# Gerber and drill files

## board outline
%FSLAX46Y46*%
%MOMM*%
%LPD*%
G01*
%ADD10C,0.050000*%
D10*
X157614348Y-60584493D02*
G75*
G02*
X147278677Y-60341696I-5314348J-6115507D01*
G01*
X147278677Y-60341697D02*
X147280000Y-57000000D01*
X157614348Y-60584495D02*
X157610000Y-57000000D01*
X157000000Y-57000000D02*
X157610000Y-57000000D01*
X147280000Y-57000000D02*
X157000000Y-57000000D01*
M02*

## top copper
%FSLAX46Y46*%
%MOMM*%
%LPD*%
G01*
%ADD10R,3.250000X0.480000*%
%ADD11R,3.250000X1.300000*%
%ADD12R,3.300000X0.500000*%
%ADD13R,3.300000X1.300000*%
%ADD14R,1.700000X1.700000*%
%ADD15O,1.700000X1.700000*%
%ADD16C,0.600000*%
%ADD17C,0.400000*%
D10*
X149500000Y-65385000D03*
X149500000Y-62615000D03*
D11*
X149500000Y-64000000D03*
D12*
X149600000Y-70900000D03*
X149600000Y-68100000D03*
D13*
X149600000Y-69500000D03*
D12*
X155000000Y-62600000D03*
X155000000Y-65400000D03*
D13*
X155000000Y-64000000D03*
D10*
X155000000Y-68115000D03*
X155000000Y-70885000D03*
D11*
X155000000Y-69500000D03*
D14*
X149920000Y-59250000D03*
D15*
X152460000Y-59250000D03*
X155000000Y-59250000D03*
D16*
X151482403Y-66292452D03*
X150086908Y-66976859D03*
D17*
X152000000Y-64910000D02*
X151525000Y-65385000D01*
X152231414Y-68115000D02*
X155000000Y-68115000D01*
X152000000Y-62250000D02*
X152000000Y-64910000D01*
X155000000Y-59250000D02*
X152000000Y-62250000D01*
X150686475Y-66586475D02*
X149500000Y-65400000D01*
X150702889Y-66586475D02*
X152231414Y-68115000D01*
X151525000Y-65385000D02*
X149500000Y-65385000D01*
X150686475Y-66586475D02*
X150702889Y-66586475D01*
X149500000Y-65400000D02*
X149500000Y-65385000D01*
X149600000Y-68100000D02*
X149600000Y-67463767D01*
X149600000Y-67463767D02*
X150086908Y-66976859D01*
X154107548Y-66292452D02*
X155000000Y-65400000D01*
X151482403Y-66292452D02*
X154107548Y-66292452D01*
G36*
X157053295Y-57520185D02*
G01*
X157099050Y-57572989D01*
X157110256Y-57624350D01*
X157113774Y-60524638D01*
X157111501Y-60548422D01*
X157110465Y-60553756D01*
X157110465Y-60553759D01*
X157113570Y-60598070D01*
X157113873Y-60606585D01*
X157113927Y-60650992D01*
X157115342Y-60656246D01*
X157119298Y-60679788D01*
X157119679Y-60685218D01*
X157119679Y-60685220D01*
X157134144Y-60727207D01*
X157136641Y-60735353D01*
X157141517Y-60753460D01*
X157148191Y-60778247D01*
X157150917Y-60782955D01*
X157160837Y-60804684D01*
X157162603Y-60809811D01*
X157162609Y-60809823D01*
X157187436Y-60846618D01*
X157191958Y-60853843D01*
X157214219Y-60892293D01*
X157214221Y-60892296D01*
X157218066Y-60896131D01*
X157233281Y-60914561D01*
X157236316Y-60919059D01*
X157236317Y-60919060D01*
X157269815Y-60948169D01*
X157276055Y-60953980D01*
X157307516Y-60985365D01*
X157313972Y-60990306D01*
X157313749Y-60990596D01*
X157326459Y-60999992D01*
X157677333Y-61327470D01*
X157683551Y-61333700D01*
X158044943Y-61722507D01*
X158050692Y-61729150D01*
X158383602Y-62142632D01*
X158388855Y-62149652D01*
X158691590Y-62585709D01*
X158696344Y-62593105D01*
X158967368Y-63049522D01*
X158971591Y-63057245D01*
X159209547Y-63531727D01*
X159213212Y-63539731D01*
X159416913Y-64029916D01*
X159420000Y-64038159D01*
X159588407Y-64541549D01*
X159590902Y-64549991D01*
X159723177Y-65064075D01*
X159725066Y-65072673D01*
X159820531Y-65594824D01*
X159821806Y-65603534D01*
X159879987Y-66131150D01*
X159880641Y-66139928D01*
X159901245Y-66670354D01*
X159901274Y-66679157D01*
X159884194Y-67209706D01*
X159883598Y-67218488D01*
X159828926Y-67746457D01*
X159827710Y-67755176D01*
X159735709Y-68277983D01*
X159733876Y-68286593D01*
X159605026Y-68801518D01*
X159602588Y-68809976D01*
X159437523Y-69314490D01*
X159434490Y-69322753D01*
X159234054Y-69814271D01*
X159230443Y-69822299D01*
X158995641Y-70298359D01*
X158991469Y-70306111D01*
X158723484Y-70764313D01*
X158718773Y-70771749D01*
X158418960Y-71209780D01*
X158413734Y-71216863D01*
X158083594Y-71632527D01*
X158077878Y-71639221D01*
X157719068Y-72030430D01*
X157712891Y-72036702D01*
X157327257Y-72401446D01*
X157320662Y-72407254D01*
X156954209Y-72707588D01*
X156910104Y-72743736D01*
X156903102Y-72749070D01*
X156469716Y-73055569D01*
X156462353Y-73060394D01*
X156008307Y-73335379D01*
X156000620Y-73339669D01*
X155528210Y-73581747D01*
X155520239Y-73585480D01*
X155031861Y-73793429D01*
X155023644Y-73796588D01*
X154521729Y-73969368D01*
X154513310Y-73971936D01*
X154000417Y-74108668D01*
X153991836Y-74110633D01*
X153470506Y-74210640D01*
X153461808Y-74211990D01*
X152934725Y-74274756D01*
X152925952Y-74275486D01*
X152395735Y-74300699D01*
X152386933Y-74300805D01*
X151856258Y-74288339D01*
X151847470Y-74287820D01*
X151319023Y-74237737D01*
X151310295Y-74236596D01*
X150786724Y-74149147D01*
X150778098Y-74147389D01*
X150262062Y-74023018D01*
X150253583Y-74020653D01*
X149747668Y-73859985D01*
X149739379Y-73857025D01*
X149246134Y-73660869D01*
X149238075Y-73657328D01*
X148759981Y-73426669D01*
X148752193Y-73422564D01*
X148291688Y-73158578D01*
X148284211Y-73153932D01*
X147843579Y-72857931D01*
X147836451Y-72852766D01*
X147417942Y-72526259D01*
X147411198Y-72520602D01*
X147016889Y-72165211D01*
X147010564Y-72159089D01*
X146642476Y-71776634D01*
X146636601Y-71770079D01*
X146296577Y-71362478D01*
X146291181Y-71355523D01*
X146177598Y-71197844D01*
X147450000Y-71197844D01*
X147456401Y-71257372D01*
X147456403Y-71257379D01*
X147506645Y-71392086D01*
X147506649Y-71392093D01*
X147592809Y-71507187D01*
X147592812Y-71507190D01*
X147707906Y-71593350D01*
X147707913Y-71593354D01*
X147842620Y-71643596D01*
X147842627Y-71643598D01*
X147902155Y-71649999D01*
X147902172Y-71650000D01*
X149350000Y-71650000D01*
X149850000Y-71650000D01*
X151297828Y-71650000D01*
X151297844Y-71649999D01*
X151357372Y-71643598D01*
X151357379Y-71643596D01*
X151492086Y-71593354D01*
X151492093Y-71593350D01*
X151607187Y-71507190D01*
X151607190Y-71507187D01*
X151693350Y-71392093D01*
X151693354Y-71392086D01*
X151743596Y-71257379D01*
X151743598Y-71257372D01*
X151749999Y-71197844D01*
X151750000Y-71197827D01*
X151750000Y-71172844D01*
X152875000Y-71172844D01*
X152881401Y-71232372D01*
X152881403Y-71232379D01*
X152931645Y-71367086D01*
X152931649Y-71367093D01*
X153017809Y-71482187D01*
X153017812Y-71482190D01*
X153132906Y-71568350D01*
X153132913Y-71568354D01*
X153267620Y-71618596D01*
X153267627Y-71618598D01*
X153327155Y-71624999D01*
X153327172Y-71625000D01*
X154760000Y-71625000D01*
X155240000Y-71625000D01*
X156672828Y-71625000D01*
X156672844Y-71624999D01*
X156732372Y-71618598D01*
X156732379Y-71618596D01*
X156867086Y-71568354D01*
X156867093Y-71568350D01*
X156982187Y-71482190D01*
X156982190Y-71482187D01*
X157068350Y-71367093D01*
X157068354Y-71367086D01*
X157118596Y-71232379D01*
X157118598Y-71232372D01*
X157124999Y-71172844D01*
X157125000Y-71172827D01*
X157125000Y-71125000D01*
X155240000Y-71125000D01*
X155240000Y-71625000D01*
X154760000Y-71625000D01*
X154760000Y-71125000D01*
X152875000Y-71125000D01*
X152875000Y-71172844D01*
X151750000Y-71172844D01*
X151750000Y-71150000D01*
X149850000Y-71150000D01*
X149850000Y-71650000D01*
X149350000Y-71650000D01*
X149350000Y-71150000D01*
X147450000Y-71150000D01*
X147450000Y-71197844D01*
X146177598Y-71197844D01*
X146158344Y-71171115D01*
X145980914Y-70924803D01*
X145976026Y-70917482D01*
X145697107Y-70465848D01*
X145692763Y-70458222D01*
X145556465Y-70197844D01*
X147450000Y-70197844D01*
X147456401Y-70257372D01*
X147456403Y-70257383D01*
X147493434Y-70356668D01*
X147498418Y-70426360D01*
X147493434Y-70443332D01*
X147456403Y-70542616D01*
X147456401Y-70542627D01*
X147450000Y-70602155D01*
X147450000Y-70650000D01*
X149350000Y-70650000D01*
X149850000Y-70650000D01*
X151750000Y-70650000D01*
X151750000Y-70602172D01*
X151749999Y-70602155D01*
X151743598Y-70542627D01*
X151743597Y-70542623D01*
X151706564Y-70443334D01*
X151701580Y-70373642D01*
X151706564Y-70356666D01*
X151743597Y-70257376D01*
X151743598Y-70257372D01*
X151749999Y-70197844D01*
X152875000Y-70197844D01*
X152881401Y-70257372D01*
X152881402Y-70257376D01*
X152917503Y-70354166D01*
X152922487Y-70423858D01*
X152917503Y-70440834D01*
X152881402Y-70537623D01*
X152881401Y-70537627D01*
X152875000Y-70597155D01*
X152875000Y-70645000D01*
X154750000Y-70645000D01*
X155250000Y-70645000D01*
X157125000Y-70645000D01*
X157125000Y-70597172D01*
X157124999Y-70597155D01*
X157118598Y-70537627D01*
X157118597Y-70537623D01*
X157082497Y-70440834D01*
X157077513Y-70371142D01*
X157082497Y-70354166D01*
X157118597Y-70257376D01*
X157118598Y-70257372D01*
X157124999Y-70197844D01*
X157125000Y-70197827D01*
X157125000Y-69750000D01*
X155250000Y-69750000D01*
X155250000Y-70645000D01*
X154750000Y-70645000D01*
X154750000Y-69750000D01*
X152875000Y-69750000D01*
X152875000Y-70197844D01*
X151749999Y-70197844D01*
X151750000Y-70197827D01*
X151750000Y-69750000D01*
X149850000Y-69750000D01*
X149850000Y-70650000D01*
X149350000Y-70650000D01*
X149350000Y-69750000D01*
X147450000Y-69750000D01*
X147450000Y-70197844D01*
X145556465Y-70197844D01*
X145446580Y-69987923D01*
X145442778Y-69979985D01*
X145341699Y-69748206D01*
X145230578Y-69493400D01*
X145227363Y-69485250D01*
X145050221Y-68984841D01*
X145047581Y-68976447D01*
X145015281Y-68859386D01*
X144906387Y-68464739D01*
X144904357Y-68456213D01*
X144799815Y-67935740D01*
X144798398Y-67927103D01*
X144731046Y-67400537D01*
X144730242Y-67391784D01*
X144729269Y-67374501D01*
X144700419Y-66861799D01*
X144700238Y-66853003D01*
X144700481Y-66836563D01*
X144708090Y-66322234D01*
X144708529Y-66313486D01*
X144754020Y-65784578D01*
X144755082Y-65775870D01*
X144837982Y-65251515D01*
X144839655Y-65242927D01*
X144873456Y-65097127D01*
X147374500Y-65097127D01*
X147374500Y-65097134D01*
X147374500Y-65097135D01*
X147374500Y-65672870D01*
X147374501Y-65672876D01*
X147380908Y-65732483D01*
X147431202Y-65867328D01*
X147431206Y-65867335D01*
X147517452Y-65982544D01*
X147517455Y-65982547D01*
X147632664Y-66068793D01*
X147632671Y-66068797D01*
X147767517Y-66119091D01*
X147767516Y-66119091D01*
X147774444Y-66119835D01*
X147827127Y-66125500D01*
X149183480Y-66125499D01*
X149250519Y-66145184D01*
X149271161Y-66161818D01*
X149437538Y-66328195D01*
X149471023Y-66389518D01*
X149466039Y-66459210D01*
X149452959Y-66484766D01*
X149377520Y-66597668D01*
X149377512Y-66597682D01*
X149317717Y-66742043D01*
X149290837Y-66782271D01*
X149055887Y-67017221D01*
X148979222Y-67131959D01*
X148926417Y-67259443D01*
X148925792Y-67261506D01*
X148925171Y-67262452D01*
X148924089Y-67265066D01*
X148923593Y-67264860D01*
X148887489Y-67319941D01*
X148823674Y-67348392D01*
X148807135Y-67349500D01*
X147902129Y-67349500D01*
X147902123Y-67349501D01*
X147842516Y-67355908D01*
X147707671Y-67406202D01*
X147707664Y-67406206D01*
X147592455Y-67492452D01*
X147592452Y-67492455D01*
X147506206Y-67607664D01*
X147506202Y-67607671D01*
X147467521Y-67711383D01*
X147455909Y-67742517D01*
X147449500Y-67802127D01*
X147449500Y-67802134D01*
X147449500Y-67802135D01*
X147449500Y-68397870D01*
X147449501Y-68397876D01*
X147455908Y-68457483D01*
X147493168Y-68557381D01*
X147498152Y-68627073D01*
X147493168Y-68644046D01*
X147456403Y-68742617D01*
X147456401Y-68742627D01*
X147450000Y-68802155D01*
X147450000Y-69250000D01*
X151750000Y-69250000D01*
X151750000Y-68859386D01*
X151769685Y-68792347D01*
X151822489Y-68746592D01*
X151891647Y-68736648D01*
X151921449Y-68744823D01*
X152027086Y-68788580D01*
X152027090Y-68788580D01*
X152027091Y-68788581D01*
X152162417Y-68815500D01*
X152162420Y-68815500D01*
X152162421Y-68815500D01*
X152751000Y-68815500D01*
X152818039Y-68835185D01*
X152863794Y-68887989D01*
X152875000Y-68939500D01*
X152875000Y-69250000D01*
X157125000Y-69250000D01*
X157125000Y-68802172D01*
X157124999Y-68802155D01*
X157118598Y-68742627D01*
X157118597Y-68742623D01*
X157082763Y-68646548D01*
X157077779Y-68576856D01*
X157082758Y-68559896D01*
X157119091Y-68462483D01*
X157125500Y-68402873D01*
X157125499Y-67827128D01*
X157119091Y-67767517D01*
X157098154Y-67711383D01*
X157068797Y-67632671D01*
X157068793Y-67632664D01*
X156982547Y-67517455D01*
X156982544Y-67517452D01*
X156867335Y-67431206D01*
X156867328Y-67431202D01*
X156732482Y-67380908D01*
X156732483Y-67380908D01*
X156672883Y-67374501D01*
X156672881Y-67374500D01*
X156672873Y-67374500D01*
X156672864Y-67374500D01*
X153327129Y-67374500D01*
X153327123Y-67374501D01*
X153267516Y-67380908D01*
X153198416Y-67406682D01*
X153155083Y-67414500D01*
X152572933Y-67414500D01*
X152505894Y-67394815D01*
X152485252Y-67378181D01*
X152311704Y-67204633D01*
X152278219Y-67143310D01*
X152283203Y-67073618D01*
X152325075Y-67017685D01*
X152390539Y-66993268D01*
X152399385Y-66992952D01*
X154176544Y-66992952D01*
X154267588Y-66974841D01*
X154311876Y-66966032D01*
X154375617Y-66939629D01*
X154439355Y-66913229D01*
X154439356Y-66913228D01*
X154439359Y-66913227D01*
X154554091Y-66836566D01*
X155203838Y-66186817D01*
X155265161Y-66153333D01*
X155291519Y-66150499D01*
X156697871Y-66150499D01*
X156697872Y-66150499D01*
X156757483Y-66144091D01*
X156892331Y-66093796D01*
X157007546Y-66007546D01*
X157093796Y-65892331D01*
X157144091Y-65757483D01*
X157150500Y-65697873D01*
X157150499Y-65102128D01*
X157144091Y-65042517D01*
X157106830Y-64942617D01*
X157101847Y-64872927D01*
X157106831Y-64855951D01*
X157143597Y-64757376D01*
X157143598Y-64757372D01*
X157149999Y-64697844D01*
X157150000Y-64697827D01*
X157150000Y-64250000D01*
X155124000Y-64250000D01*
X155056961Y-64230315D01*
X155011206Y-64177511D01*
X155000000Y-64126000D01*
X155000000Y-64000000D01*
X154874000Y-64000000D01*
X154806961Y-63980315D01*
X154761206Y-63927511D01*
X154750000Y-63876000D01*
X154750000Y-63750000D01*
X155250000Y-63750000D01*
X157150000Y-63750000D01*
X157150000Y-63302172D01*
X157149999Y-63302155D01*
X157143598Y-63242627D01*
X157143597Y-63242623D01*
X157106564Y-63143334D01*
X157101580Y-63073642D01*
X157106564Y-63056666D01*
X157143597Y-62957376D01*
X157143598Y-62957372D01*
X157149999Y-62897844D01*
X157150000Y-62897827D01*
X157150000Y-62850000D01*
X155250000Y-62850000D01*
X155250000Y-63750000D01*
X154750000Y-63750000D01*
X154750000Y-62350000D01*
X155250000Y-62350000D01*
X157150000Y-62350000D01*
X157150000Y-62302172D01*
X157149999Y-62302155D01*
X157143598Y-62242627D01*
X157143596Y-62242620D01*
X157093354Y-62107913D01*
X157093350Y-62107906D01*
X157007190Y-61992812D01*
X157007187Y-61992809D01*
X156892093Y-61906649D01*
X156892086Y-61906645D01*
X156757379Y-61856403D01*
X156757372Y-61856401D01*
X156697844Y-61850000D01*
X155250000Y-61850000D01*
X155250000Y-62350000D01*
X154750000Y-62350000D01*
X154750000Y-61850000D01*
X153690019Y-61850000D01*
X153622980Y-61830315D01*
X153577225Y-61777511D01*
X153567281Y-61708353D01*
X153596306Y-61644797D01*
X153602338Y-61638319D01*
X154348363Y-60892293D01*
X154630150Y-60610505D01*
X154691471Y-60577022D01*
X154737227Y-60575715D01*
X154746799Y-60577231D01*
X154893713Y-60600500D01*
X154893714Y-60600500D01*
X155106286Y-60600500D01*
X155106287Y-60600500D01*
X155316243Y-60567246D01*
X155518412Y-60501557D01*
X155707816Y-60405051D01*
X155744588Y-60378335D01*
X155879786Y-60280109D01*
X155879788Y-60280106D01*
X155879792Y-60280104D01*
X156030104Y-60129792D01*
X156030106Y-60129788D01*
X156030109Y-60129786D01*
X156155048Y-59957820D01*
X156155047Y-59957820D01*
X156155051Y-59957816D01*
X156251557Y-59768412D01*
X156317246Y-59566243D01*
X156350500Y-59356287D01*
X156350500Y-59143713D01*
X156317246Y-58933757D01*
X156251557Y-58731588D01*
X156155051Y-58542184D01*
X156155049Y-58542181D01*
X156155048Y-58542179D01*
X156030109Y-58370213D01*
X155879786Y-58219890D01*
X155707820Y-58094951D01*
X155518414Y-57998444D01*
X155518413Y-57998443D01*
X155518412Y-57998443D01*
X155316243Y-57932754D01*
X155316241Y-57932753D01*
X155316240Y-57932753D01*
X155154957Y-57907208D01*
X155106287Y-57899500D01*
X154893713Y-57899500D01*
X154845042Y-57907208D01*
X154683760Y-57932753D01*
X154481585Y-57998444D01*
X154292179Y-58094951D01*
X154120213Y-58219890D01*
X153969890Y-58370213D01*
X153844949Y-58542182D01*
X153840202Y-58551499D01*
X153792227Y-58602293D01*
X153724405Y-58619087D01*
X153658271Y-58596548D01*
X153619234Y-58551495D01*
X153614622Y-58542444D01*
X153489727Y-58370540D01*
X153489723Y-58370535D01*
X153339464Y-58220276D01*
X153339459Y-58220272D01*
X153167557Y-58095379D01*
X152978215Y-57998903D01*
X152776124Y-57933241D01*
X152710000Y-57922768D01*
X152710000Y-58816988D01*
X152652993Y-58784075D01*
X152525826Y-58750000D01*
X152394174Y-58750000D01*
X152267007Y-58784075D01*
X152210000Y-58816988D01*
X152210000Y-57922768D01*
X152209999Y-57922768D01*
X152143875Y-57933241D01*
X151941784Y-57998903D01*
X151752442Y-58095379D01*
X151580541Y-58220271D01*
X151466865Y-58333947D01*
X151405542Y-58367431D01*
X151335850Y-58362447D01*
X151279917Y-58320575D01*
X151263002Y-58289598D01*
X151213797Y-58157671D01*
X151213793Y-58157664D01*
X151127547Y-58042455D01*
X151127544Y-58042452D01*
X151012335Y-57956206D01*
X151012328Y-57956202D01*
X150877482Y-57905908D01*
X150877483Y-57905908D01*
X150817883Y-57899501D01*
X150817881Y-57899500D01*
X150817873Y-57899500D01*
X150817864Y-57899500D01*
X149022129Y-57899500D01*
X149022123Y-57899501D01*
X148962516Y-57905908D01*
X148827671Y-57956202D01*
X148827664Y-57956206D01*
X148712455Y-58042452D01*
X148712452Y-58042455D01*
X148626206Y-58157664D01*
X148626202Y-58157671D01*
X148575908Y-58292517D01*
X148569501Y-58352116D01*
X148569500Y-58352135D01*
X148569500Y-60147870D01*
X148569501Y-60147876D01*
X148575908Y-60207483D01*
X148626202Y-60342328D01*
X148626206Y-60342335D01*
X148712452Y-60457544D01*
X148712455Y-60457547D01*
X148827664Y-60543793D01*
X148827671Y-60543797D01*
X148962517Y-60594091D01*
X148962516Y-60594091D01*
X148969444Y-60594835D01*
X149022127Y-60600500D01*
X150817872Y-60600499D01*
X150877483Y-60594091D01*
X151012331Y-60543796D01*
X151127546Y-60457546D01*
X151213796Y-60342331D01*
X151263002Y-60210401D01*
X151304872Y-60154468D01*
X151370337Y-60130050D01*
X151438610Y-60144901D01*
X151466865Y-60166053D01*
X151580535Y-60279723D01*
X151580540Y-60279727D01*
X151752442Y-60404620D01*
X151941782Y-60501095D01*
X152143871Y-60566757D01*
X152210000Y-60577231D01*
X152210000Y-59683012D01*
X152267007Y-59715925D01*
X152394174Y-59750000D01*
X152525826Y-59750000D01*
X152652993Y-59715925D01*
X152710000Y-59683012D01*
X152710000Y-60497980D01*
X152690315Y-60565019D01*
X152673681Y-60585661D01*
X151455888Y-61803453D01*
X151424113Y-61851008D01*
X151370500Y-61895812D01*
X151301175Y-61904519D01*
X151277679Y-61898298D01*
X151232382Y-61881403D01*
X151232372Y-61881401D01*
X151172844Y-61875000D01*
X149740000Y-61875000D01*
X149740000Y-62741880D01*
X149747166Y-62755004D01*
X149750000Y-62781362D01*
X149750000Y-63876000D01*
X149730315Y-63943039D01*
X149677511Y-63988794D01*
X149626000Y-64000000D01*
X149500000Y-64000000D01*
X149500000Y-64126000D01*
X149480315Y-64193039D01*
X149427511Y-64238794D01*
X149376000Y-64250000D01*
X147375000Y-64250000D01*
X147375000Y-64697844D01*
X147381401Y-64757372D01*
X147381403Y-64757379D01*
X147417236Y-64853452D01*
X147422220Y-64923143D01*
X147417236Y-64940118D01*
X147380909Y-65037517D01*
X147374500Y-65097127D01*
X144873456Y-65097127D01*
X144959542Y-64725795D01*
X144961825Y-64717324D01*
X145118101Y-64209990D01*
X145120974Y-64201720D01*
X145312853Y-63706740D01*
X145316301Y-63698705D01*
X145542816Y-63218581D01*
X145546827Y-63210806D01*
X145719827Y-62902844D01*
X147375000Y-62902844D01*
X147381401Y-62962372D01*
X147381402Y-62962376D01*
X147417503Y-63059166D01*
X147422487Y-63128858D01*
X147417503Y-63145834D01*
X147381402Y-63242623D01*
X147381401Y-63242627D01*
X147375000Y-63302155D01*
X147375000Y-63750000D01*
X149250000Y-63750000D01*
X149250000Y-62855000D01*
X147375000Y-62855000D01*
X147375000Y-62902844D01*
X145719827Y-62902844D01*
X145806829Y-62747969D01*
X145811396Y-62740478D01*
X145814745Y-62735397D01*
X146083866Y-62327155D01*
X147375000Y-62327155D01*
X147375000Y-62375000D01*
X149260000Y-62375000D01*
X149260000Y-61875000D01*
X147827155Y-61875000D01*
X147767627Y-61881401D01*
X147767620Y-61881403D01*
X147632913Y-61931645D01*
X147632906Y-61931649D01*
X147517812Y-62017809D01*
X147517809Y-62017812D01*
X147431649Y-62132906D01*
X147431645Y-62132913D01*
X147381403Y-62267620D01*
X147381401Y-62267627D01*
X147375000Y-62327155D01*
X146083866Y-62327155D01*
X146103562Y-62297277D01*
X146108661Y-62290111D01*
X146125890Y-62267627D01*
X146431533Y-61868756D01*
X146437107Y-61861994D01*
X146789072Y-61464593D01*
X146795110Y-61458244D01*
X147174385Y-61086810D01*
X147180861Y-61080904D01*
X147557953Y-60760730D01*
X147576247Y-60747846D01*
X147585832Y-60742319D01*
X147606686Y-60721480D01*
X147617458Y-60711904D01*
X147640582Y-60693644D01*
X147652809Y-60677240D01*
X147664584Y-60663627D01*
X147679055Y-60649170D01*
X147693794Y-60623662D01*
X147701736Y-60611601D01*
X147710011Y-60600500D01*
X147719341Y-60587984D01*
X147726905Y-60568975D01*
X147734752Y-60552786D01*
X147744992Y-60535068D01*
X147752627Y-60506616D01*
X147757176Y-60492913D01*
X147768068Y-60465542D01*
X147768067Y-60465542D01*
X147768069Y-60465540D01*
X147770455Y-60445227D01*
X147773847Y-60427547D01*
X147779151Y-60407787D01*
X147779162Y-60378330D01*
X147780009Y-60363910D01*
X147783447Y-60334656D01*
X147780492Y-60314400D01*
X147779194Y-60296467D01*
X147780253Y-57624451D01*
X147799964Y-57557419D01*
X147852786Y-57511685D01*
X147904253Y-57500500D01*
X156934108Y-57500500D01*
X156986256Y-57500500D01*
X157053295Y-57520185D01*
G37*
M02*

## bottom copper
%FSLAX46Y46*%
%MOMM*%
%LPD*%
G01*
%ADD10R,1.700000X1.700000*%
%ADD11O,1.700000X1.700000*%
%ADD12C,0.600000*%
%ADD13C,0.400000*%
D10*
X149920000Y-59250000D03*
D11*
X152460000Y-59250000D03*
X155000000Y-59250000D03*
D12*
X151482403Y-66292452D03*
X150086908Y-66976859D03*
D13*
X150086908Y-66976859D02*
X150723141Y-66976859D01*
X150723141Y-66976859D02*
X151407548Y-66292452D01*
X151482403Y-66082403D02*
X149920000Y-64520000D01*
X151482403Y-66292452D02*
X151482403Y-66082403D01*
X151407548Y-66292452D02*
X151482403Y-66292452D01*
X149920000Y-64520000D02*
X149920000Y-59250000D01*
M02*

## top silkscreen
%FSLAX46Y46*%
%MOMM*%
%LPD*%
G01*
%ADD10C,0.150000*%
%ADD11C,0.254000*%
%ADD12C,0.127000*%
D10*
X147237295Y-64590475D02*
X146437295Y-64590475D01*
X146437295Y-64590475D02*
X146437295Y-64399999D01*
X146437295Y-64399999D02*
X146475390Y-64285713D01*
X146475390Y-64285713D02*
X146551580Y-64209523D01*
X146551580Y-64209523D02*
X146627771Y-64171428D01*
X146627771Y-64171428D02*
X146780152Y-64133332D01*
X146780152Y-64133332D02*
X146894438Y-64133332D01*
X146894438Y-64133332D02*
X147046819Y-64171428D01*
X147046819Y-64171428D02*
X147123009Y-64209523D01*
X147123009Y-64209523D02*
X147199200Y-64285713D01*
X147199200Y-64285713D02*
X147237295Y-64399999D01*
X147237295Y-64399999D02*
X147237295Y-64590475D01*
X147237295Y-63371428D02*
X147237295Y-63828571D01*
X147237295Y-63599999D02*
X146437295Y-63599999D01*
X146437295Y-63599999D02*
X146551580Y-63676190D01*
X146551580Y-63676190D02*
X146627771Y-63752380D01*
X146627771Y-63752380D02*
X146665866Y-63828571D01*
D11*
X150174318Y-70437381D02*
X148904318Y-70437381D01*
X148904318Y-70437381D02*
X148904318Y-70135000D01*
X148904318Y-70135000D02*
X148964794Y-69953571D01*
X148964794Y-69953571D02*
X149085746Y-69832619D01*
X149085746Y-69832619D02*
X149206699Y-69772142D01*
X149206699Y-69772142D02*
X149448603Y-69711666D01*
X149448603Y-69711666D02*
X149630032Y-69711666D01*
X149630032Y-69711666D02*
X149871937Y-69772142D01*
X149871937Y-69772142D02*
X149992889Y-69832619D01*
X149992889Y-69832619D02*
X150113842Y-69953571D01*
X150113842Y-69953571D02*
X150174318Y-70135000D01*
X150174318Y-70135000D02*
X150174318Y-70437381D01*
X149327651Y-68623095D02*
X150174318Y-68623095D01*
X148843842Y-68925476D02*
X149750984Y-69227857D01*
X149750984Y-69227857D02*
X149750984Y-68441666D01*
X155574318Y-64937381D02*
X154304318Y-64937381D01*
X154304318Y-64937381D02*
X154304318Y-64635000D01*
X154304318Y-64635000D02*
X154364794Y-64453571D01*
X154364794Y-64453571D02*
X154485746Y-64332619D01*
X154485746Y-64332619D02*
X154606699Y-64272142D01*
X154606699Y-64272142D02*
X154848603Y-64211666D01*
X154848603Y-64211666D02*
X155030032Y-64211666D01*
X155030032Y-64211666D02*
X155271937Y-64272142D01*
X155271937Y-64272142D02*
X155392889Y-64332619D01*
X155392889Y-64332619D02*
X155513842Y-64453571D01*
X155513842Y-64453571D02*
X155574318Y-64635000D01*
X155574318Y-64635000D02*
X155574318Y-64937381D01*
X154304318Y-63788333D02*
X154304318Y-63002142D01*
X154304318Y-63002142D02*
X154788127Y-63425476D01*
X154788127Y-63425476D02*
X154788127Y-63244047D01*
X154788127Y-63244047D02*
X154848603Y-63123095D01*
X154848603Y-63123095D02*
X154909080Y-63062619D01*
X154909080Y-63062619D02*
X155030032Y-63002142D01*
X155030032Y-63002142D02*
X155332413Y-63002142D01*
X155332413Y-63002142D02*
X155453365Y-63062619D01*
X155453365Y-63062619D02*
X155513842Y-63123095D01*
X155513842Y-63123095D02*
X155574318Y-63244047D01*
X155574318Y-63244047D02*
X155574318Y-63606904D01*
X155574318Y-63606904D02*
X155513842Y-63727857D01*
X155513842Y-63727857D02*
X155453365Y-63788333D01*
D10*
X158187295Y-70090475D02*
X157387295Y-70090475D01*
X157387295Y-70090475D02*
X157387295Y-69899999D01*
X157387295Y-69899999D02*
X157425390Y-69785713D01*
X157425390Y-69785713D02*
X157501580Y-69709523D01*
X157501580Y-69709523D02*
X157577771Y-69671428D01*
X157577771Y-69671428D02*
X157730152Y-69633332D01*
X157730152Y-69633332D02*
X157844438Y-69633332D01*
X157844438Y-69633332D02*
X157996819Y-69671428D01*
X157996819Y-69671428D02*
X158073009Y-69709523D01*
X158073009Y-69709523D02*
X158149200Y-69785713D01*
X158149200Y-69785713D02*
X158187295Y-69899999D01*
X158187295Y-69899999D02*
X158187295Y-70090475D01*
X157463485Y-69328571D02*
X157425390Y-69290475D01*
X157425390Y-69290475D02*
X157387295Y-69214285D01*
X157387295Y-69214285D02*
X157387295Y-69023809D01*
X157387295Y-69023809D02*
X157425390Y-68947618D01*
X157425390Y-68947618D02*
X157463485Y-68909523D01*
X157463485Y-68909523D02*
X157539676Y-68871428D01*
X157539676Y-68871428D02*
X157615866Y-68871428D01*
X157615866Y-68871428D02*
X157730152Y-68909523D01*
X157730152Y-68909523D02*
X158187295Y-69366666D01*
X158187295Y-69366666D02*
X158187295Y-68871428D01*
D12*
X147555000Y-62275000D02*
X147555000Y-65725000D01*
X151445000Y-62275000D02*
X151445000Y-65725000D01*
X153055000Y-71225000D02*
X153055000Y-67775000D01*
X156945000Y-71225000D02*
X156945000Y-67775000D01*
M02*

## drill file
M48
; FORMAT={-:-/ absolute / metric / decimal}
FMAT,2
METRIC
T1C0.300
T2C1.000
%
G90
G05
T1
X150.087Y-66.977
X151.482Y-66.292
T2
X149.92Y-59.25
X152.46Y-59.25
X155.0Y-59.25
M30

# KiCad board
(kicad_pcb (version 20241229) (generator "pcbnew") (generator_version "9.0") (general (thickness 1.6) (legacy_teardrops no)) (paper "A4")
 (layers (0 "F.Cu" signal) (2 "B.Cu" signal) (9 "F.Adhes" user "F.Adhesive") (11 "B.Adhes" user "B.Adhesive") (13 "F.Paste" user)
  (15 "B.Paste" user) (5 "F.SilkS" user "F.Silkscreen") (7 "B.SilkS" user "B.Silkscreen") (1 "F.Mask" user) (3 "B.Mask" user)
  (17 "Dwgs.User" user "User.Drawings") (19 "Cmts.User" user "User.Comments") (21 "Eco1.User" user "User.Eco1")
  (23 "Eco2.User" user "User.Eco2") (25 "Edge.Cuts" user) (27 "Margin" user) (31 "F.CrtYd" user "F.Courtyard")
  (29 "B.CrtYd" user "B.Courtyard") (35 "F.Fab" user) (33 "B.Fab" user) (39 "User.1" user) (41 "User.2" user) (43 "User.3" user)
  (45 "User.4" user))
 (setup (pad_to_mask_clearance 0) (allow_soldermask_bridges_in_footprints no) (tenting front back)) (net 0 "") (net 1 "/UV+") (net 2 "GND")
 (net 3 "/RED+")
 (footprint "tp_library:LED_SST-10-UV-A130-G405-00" (layer "F.Cu") (at 149.5 64 -90)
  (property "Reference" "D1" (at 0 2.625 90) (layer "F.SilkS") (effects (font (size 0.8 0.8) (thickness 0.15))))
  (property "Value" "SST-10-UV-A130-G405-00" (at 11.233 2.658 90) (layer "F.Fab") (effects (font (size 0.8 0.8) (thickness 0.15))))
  (fp_line (start -1.725 1.945) (end 1.725 1.945) (stroke (width 0.127) (type solid)) (layer "F.SilkS"))
  (fp_line (start -1.725 -1.945) (end 1.725 -1.945) (stroke (width 0.127) (type solid)) (layer "F.SilkS"))
  (pad "A" smd rect (at 1.385 0 270) (size 0.48 3.25) (layers "F.Cu" "F.Mask" "F.Paste") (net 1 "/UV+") (solder_mask_margin 0.102))
  (pad "C" smd rect (at -1.385 0 270) (size 0.48 3.25) (layers "F.Cu" "F.Mask" "F.Paste") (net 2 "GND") (solder_mask_margin 0.102))
  (pad "S" smd rect (at 0 0 270) (size 1.3 3.25) (layers "F.Cu" "F.Mask") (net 2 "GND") (solder_mask_margin 0.102)))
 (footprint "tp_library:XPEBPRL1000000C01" (layer "F.Cu") (at 149.6 69.5 90)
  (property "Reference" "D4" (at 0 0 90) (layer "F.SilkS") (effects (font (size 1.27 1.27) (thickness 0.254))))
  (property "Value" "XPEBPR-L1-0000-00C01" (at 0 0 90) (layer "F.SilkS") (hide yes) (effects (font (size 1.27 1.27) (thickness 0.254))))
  (pad "1" smd rect (at -1.4 0 90) (size 0.5 3.3) (layers "F.Cu" "F.Mask" "F.Paste") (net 2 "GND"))
  (pad "2" smd rect (at 1.4 0 90) (size 0.5 3.3) (layers "F.Cu" "F.Mask" "F.Paste") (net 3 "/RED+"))
  (pad "3" smd rect (at 0 0 90) (size 1.3 3.3) (layers "F.Cu" "F.Mask" "F.Paste") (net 2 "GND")))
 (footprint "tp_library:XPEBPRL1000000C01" (layer "F.Cu") (at 155 64 -90)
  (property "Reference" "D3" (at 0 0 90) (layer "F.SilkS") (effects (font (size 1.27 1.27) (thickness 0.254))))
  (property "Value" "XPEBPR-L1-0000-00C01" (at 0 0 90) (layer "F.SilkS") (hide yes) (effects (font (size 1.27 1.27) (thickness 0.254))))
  (pad "1" smd rect (at -1.4 0 270) (size 0.5 3.3) (layers "F.Cu" "F.Mask" "F.Paste") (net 2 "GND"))
  (pad "2" smd rect (at 1.4 0 270) (size 0.5 3.3) (layers "F.Cu" "F.Mask" "F.Paste") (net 3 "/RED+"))
  (pad "3" smd rect (at 0 0 270) (size 1.3 3.3) (layers "F.Cu" "F.Mask" "F.Paste") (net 2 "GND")))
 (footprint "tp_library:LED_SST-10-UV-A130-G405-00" (layer "F.Cu") (at 155 69.5 90)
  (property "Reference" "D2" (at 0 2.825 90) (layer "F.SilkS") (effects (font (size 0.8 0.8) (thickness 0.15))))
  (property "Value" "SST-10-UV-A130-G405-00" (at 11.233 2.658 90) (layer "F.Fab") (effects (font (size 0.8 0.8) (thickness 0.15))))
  (fp_line (start -1.725 -1.945) (end 1.725 -1.945) (stroke (width 0.127) (type solid)) (layer "F.SilkS"))
  (fp_line (start -1.725 1.945) (end 1.725 1.945) (stroke (width 0.127) (type solid)) (layer "F.SilkS"))
  (pad "A" smd rect (at 1.385 0 90) (size 0.48 3.25) (layers "F.Cu" "F.Mask" "F.Paste") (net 1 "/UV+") (solder_mask_margin 0.102))
  (pad "C" smd rect (at -1.385 0 90) (size 0.48 3.25) (layers "F.Cu" "F.Mask" "F.Paste") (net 2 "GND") (solder_mask_margin 0.102))
  (pad "S" smd rect (at 0 0 90) (size 1.3 3.25) (layers "F.Cu" "F.Mask") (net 2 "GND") (solder_mask_margin 0.102)))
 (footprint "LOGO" (layer "B.Cu") (at 152.3 66.8 90)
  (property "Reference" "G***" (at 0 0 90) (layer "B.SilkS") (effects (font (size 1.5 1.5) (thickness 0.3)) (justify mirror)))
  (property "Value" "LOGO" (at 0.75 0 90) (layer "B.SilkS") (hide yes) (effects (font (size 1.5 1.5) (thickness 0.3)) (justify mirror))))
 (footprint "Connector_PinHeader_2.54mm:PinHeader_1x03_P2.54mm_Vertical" (layer "B.Cu") (at 149.92 59.25 -90)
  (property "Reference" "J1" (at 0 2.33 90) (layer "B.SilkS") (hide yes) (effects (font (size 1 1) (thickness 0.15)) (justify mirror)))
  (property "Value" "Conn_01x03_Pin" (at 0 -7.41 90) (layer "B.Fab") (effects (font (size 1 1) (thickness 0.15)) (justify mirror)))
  (pad "1" thru_hole rect (at 0 0 270) (size 1.7 1.7) (drill 1) (layers "*.Cu" "*.Mask") (remove_unused_layers no) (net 3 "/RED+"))
  (pad "2" thru_hole oval (at 0 -2.54 270) (size 1.7 1.7) (drill 1) (layers "*.Cu" "*.Mask") (remove_unused_layers no) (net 2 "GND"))
  (pad "3" thru_hole oval (at 0 -5.08 270) (size 1.7 1.7) (drill 1) (layers "*.Cu" "*.Mask") (remove_unused_layers no) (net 1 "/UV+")))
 (gr_arc (start 157.614348 60.584493) (mid 152.109728 74.799723) (end 147.278677 60.341696) (stroke (width 0.05) (type default))
  (layer "Edge.Cuts"))
 (gr_line (start 147.278677 60.341697) (end 147.28 57) (stroke (width 0.05) (type default)) (layer "Edge.Cuts"))
 (gr_line (start 157.614348 60.584495) (end 157.61 57) (stroke (width 0.05) (type default)) (layer "Edge.Cuts"))
 (gr_line (start 157 57) (end 157.61 57) (stroke (width 0.05) (type default)) (layer "Edge.Cuts"))
 (gr_line (start 147.28 57) (end 157 57) (stroke (width 0.05) (type default)) (layer "Edge.Cuts"))
 (segment (start 152 64.91) (end 151.525 65.385) (width 0.4) (layer "F.Cu") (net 1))
 (segment (start 152.231414 68.115) (end 155 68.115) (width 0.4) (layer "F.Cu") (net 1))
 (segment (start 152 62.25) (end 152 64.91) (width 0.4) (layer "F.Cu") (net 1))
 (segment (start 155 59.25) (end 152 62.25) (width 0.4) (layer "F.Cu") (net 1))
 (segment (start 150.686475 66.586475) (end 149.5 65.4) (width 0.4) (layer "F.Cu") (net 1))
 (segment (start 150.702889 66.586475) (end 152.231414 68.115) (width 0.4) (layer "F.Cu") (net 1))
 (segment (start 151.525 65.385) (end 149.5 65.385) (width 0.4) (layer "F.Cu") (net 1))
 (segment (start 150.686475 66.586475) (end 150.702889 66.586475) (width 0.4) (layer "F.Cu") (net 1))
 (segment (start 149.5 65.4) (end 149.5 65.385) (width 0.4) (layer "F.Cu") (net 1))
 (segment (start 149.6 68.1) (end 149.6 67.463767) (width 0.4) (layer "F.Cu") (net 3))
 (segment (start 149.6 67.463767) (end 150.086908 66.976859) (width 0.4) (layer "F.Cu") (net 3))
 (segment (start 154.107548 66.292452) (end 155 65.4) (width 0.4) (layer "F.Cu") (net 3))
 (segment (start 151.482403 66.292452) (end 154.107548 66.292452) (width 0.4) (layer "F.Cu") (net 3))
 (via (at 151.482403 66.292452) (size 0.6) (drill 0.3) (layers "F.Cu" "B.Cu") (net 3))
 (via (at 150.086908 66.976859) (size 0.6) (drill 0.3) (layers "F.Cu" "B.Cu") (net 3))
 (segment (start 150.086908 66.976859) (end 150.723141 66.976859) (width 0.4) (layer "B.Cu") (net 3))
 (segment (start 150.723141 66.976859) (end 151.407548 66.292452) (width 0.4) (layer "B.Cu") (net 3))
 (segment (start 151.482403 66.082403) (end 149.92 64.52) (width 0.4) (layer "B.Cu") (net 3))
 (segment (start 151.482403 66.292452) (end 151.482403 66.082403) (width 0.4) (layer "B.Cu") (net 3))
 (segment (start 151.407548 66.292452) (end 151.482403 66.292452) (width 0.4) (layer "B.Cu") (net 3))
 (segment (start 149.92 64.52) (end 149.92 59.25) (width 0.4) (layer "B.Cu") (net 3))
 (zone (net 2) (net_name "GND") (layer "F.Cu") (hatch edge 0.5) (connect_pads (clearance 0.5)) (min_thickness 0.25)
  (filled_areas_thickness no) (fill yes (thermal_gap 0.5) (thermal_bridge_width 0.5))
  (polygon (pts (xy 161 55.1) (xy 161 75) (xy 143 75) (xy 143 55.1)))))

